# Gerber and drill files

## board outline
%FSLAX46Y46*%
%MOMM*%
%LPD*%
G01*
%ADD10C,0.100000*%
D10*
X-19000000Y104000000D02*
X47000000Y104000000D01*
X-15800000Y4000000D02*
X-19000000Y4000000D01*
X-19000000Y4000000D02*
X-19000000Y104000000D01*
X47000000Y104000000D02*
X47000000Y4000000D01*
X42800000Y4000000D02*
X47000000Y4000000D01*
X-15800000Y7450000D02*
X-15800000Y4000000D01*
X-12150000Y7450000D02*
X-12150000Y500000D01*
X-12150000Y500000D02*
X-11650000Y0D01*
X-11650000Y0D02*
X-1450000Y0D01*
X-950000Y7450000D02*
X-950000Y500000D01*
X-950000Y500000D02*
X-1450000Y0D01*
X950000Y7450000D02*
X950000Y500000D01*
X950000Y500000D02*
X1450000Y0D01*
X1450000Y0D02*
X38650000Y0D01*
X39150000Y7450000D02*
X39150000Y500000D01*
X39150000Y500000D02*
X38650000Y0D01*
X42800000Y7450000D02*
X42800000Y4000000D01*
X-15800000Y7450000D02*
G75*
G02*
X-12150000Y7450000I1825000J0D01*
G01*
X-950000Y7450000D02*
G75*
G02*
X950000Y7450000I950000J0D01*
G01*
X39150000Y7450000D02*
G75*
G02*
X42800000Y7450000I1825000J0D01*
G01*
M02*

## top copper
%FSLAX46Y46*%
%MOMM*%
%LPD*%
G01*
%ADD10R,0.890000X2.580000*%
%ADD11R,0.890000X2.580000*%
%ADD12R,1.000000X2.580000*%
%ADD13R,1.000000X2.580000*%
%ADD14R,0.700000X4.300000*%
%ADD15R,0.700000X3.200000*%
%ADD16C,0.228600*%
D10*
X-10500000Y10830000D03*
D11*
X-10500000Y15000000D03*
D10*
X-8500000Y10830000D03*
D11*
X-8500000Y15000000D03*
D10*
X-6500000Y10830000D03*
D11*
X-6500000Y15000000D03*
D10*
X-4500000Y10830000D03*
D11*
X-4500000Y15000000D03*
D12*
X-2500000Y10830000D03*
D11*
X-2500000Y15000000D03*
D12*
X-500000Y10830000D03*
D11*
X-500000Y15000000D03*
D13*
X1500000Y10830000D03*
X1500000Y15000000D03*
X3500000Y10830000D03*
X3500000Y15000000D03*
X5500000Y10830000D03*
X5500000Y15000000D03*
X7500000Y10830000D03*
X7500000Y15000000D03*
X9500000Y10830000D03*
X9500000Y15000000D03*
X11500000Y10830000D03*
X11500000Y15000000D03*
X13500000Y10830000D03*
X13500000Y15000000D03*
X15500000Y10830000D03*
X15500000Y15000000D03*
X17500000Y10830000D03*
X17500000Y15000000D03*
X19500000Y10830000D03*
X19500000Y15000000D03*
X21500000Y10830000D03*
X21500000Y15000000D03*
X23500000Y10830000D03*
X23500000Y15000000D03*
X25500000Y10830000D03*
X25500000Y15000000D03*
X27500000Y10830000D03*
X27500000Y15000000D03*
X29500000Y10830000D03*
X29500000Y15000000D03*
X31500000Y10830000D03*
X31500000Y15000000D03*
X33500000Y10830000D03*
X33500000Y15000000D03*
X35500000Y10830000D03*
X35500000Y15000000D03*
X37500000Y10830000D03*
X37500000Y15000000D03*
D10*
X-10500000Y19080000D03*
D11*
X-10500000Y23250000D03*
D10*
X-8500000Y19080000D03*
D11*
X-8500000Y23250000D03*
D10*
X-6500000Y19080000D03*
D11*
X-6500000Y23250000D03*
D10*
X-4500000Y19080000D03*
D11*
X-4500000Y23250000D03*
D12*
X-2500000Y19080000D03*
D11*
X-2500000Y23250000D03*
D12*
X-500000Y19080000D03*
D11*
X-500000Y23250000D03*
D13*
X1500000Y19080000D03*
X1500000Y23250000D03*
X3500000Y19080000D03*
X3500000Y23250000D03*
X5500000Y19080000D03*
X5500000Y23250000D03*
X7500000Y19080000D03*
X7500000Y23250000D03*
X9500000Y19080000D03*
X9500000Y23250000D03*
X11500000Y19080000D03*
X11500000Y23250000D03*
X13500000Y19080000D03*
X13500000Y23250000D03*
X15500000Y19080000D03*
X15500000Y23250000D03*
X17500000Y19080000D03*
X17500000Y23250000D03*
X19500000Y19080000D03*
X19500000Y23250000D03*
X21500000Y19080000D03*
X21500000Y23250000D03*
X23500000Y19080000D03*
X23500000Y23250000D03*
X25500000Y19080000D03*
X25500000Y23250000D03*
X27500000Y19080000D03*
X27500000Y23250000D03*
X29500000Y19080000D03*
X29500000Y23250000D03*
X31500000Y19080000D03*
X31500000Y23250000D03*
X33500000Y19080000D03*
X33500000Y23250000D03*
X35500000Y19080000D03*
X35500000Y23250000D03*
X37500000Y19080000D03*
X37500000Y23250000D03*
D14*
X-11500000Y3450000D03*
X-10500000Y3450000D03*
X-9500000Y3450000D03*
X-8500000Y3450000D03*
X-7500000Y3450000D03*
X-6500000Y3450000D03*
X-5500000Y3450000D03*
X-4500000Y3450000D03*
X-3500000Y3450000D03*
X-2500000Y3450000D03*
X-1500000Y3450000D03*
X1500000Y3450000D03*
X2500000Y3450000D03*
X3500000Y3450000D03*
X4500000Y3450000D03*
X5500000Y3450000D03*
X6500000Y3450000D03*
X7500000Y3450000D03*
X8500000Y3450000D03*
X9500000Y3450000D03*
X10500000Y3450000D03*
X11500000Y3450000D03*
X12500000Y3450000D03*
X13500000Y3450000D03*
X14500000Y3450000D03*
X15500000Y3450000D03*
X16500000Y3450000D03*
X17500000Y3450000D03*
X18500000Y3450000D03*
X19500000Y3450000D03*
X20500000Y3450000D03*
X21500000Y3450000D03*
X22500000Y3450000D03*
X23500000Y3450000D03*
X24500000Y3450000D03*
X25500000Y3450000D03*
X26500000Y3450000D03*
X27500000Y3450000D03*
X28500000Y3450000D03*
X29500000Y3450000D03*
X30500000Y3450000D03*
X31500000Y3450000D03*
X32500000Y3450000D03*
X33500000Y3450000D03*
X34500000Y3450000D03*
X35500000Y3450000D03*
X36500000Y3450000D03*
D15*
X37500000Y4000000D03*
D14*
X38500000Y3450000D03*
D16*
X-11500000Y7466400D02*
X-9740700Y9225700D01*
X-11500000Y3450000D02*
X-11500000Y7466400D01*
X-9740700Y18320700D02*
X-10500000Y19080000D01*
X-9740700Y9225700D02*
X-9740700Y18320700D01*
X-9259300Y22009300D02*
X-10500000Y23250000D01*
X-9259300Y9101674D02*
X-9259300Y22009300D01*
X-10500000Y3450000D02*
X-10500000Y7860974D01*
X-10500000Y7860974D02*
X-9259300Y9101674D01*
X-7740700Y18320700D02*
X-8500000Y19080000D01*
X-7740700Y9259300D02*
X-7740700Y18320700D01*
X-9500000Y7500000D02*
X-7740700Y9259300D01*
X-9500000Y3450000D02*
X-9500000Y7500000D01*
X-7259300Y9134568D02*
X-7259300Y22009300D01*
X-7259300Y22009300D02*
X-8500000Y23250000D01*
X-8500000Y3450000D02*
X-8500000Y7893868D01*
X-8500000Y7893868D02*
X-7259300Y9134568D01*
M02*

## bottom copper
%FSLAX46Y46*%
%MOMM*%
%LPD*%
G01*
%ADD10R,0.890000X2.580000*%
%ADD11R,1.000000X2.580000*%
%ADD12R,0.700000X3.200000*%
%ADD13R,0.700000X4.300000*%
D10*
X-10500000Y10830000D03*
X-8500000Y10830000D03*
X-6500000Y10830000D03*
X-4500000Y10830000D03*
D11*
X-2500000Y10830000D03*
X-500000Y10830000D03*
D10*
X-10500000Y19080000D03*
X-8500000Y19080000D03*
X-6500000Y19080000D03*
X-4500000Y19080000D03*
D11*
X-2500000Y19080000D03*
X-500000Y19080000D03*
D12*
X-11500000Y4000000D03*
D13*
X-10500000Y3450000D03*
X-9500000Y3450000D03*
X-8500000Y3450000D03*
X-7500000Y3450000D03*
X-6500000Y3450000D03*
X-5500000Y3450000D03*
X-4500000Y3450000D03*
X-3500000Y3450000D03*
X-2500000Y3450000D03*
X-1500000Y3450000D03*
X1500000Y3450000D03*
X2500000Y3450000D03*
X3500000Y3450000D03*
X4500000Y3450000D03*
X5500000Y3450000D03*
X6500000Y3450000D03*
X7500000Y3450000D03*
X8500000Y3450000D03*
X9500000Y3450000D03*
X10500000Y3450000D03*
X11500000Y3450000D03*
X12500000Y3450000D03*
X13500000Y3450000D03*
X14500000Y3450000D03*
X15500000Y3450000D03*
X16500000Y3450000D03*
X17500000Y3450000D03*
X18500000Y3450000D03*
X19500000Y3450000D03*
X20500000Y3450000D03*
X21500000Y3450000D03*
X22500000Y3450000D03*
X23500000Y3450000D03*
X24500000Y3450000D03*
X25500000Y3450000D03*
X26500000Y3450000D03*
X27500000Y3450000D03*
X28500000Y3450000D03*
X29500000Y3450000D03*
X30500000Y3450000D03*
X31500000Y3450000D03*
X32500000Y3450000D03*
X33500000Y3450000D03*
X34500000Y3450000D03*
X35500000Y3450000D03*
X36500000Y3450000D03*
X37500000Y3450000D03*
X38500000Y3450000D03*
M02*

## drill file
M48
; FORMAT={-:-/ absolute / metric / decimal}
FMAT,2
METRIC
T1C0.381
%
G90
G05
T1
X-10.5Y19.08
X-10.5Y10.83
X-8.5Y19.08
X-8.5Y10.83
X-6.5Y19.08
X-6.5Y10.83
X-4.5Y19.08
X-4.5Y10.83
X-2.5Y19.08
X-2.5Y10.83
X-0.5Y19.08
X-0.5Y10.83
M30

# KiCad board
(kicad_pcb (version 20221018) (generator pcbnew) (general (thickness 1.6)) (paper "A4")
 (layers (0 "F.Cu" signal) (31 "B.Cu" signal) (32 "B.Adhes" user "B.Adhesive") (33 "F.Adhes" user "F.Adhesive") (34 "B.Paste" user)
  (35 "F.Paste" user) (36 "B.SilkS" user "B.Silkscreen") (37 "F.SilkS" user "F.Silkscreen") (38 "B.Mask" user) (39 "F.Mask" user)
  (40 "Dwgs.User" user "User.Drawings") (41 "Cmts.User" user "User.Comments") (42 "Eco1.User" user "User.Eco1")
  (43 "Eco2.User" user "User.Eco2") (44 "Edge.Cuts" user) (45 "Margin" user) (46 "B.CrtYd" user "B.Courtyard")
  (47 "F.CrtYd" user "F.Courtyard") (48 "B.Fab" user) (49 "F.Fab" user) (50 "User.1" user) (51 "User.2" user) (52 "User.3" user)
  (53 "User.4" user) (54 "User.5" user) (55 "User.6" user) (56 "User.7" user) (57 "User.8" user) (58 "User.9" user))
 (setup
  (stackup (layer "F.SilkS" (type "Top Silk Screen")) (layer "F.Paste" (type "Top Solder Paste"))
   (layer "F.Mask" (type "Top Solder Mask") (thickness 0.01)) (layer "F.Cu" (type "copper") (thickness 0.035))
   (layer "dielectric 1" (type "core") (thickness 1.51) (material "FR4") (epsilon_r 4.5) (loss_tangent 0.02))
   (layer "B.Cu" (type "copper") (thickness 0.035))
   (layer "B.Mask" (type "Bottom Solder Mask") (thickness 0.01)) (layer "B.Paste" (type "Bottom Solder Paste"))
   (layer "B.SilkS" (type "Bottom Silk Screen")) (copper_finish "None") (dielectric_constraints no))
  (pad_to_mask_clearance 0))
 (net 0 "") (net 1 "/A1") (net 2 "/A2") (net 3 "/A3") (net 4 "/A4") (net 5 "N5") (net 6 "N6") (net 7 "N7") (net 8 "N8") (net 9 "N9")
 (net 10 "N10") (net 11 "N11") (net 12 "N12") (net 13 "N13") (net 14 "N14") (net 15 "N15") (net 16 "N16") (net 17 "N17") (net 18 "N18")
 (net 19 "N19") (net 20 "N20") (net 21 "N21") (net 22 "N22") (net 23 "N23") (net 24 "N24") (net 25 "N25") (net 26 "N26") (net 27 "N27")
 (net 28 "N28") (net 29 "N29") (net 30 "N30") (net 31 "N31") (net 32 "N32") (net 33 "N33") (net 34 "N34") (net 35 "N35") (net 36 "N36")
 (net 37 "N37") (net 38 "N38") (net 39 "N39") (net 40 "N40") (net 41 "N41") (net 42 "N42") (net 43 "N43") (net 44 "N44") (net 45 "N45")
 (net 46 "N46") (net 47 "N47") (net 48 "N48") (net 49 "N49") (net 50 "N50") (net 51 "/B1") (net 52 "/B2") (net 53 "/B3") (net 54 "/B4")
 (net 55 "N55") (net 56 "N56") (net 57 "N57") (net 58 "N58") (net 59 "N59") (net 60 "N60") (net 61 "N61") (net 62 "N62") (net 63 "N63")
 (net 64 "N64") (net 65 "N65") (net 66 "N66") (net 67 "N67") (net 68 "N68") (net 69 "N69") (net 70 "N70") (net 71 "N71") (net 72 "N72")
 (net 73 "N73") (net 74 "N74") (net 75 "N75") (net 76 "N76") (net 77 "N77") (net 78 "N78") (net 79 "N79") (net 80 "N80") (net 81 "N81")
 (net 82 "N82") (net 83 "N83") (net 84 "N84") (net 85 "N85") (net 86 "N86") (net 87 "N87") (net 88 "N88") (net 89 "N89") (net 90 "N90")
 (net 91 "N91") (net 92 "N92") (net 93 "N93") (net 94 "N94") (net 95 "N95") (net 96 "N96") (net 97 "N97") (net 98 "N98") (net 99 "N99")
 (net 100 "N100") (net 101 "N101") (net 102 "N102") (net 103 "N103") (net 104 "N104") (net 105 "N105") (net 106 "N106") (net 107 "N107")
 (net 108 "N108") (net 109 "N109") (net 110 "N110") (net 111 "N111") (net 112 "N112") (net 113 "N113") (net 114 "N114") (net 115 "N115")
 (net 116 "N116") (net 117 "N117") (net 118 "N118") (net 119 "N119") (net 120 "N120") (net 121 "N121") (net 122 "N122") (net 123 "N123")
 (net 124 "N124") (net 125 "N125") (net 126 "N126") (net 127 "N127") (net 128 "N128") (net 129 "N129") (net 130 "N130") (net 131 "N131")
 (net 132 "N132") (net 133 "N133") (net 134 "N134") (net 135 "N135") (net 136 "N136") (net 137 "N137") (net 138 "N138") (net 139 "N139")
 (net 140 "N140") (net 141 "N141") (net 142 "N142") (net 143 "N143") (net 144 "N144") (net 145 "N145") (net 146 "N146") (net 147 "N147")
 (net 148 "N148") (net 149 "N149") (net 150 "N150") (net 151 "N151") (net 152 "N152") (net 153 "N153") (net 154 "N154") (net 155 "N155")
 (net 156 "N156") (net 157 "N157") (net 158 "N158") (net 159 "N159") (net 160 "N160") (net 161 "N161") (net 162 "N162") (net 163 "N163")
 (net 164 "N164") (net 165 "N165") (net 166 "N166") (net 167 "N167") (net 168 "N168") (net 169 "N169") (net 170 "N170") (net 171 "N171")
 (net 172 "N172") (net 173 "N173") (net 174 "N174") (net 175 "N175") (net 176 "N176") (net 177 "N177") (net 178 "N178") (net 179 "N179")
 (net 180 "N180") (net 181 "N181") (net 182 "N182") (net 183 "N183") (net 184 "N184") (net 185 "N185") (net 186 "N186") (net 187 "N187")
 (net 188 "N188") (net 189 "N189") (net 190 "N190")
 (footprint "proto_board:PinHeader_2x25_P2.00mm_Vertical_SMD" (layer "F.Cu") (at 13.5 -12.915 90)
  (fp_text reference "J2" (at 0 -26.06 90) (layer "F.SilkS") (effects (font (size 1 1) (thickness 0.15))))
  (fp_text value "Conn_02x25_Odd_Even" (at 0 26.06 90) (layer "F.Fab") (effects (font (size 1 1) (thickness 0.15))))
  (pad "1" thru_hole rect (at -2.085 -24 90) (size 2.58 0.89) (drill 0.381) (layers "*.Cu" "*.Mask") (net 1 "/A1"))
  (pad "2" smd rect (at 2.085 -24 90) (size 2.58 0.89) (layers "F.Cu" "F.Paste" "F.Mask") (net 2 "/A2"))
  (pad "3" thru_hole rect (at -2.085 -22 90) (size 2.58 0.89) (drill 0.381) (layers "*.Cu" "*.Mask") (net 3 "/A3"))
  (pad "4" smd rect (at 2.085 -22 90) (size 2.58 0.89) (layers "F.Cu" "F.Paste" "F.Mask") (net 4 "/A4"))
  (pad "5" thru_hole rect (at -2.085 -20 90) (size 2.58 0.89) (drill 0.381) (layers "*.Cu" "*.Mask") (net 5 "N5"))
  (pad "6" smd rect (at 2.085 -20 90) (size 2.58 0.89) (layers "F.Cu" "F.Paste" "F.Mask") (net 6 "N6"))
  (pad "7" thru_hole rect (at -2.085 -18 90) (size 2.58 0.89) (drill 0.381) (layers "*.Cu" "*.Mask") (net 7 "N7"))
  (pad "8" smd rect (at 2.085 -18 90) (size 2.58 0.89) (layers "F.Cu" "F.Paste" "F.Mask") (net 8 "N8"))
  (pad "9" thru_hole rect (at -2.085 -16 90) (size 2.58 1) (drill 0.381) (layers "*.Cu" "*.Mask") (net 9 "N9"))
  (pad "10" smd rect (at 2.085 -16 90) (size 2.58 0.89) (layers "F.Cu" "F.Paste" "F.Mask") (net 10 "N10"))
  (pad "11" thru_hole rect (at -2.085 -14 90) (size 2.58 1) (drill 0.381) (layers "*.Cu" "*.Mask") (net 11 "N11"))
  (pad "12" smd rect (at 2.085 -14 90) (size 2.58 0.89) (layers "F.Cu" "F.Paste" "F.Mask") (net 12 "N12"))
  (pad "13" smd rect (at -2.085 -12 90) (size 2.58 1) (layers "F.Cu" "F.Paste" "F.Mask") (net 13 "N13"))
  (pad "14" smd rect (at 2.085 -12 90) (size 2.58 1) (layers "F.Cu" "F.Paste" "F.Mask") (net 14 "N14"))
  (pad "15" smd rect (at -2.085 -10 90) (size 2.58 1) (layers "F.Cu" "F.Paste" "F.Mask") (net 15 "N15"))
  (pad "16" smd rect (at 2.085 -10 90) (size 2.58 1) (layers "F.Cu" "F.Paste" "F.Mask") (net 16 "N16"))
  (pad "17" smd rect (at -2.085 -8 90) (size 2.58 1) (layers "F.Cu" "F.Paste" "F.Mask") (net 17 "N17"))
  (pad "18" smd rect (at 2.085 -8 90) (size 2.58 1) (layers "F.Cu" "F.Paste" "F.Mask") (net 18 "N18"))
  (pad "19" smd rect (at -2.085 -6 90) (size 2.58 1) (layers "F.Cu" "F.Paste" "F.Mask") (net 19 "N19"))
  (pad "20" smd rect (at 2.085 -6 90) (size 2.58 1) (layers "F.Cu" "F.Paste" "F.Mask") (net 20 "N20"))
  (pad "21" smd rect (at -2.085 -4 90) (size 2.58 1) (layers "F.Cu" "F.Paste" "F.Mask") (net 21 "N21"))
  (pad "22" smd rect (at 2.085 -4 90) (size 2.58 1) (layers "F.Cu" "F.Paste" "F.Mask") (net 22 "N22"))
  (pad "23" smd rect (at -2.085 -2 90) (size 2.58 1) (layers "F.Cu" "F.Paste" "F.Mask") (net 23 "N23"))
  (pad "24" smd rect (at 2.085 -2 90) (size 2.58 1) (layers "F.Cu" "F.Paste" "F.Mask") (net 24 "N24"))
  (pad "25" smd rect (at -2.085 0 90) (size 2.58 1) (layers "F.Cu" "F.Paste" "F.Mask") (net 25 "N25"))
  (pad "26" smd rect (at 2.085 0 90) (size 2.58 1) (layers "F.Cu" "F.Paste" "F.Mask") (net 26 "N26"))
  (pad "27" smd rect (at -2.085 2 90) (size 2.58 1) (layers "F.Cu" "F.Paste" "F.Mask") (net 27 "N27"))
  (pad "28" smd rect (at 2.085 2 90) (size 2.58 1) (layers "F.Cu" "F.Paste" "F.Mask") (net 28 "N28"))
  (pad "29" smd rect (at -2.085 4 90) (size 2.58 1) (layers "F.Cu" "F.Paste" "F.Mask") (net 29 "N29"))
  (pad "30" smd rect (at 2.085 4 90) (size 2.58 1) (layers "F.Cu" "F.Paste" "F.Mask") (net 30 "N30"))
  (pad "31" smd rect (at -2.085 6 90) (size 2.58 1) (layers "F.Cu" "F.Paste" "F.Mask") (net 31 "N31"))
  (pad "32" smd rect (at 2.085 6 90) (size 2.58 1) (layers "F.Cu" "F.Paste" "F.Mask") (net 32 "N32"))
  (pad "33" smd rect (at -2.085 8 90) (size 2.58 1) (layers "F.Cu" "F.Paste" "F.Mask") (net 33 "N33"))
  (pad "34" smd rect (at 2.085 8 90) (size 2.58 1) (layers "F.Cu" "F.Paste" "F.Mask") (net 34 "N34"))
  (pad "35" smd rect (at -2.085 10 90) (size 2.58 1) (layers "F.Cu" "F.Paste" "F.Mask") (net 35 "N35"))
  (pad "36" smd rect (at 2.085 10 90) (size 2.58 1) (layers "F.Cu" "F.Paste" "F.Mask") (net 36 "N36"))
  (pad "37" smd rect (at -2.085 12 90) (size 2.58 1) (layers "F.Cu" "F.Paste" "F.Mask") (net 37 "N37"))
  (pad "38" smd rect (at 2.085 12 90) (size 2.58 1) (layers "F.Cu" "F.Paste" "F.Mask") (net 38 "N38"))
  (pad "39" smd rect (at -2.085 14 90) (size 2.58 1) (layers "F.Cu" "F.Paste" "F.Mask") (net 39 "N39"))
  (pad "40" smd rect (at 2.085 14 90) (size 2.58 1) (layers "F.Cu" "F.Paste" "F.Mask") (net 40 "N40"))
  (pad "41" smd rect (at -2.085 16 90) (size 2.58 1) (layers "F.Cu" "F.Paste" "F.Mask") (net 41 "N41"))
  (pad "42" smd rect (at 2.085 16 90) (size 2.58 1) (layers "F.Cu" "F.Paste" "F.Mask") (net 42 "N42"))
  (pad "43" smd rect (at -2.085 18 90) (size 2.58 1) (layers "F.Cu" "F.Paste" "F.Mask") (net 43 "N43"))
  (pad "44" smd rect (at 2.085 18 90) (size 2.58 1) (layers "F.Cu" "F.Paste" "F.Mask") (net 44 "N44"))
  (pad "45" smd rect (at -2.085 20 90) (size 2.58 1) (layers "F.Cu" "F.Paste" "F.Mask") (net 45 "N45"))
  (pad "46" smd rect (at 2.085 20 90) (size 2.58 1) (layers "F.Cu" "F.Paste" "F.Mask") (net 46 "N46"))
  (pad "47" smd rect (at -2.085 22 90) (size 2.58 1) (layers "F.Cu" "F.Paste" "F.Mask") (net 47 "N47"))
  (pad "48" smd rect (at 2.085 22 90) (size 2.58 1) (layers "F.Cu" "F.Paste" "F.Mask") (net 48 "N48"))
  (pad "49" smd rect (at -2.085 24 90) (size 2.58 1) (layers "F.Cu" "F.Paste" "F.Mask") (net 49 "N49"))
  (pad "50" smd rect (at 2.085 24 90) (size 2.58 1) (layers "F.Cu" "F.Paste" "F.Mask") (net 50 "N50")))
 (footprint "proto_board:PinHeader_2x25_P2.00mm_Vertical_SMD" (layer "F.Cu") (at 13.5 -21.165 90)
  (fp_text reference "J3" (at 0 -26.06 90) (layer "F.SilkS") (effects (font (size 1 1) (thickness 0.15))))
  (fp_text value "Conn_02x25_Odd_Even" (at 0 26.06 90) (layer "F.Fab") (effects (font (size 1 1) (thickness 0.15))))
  (pad "1" thru_hole rect (at -2.085 -24 90) (size 2.58 0.89) (drill 0.381) (layers "*.Cu" "*.Mask") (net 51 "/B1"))
  (pad "2" smd rect (at 2.085 -24 90) (size 2.58 0.89) (layers "F.Cu" "F.Paste" "F.Mask") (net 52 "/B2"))
  (pad "3" thru_hole rect (at -2.085 -22 90) (size 2.58 0.89) (drill 0.381) (layers "*.Cu" "*.Mask") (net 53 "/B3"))
  (pad "4" smd rect (at 2.085 -22 90) (size 2.58 0.89) (layers "F.Cu" "F.Paste" "F.Mask") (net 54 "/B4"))
  (pad "5" thru_hole rect (at -2.085 -20 90) (size 2.58 0.89) (drill 0.381) (layers "*.Cu" "*.Mask") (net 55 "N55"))
  (pad "6" smd rect (at 2.085 -20 90) (size 2.58 0.89) (layers "F.Cu" "F.Paste" "F.Mask") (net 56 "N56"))
  (pad "7" thru_hole rect (at -2.085 -18 90) (size 2.58 0.89) (drill 0.381) (layers "*.Cu" "*.Mask") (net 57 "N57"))
  (pad "8" smd rect (at 2.085 -18 90) (size 2.58 0.89) (layers "F.Cu" "F.Paste" "F.Mask") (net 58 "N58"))
  (pad "9" thru_hole rect (at -2.085 -16 90) (size 2.58 1) (drill 0.381) (layers "*.Cu" "*.Mask") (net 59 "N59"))
  (pad "10" smd rect (at 2.085 -16 90) (size 2.58 0.89) (layers "F.Cu" "F.Paste" "F.Mask") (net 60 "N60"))
  (pad "11" thru_hole rect (at -2.085 -14 90) (size 2.58 1) (drill 0.381) (layers "*.Cu" "*.Mask") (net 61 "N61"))
  (pad "12" smd rect (at 2.085 -14 90) (size 2.58 0.89) (layers "F.Cu" "F.Paste" "F.Mask") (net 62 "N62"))
  (pad "13" smd rect (at -2.085 -12 90) (size 2.58 1) (layers "F.Cu" "F.Paste" "F.Mask") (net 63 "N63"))
  (pad "14" smd rect (at 2.085 -12 90) (size 2.58 1) (layers "F.Cu" "F.Paste" "F.Mask") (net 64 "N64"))
  (pad "15" smd rect (at -2.085 -10 90) (size 2.58 1) (layers "F.Cu" "F.Paste" "F.Mask") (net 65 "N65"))
  (pad "16" smd rect (at 2.085 -10 90) (size 2.58 1) (layers "F.Cu" "F.Paste" "F.Mask") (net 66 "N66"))
  (pad "17" smd rect (at -2.085 -8 90) (size 2.58 1) (layers "F.Cu" "F.Paste" "F.Mask") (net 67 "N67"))
  (pad "18" smd rect (at 2.085 -8 90) (size 2.58 1) (layers "F.Cu" "F.Paste" "F.Mask") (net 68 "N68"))
  (pad "19" smd rect (at -2.085 -6 90) (size 2.58 1) (layers "F.Cu" "F.Paste" "F.Mask") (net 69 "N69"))
  (pad "20" smd rect (at 2.085 -6 90) (size 2.58 1) (layers "F.Cu" "F.Paste" "F.Mask") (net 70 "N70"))
  (pad "21" smd rect (at -2.085 -4 90) (size 2.58 1) (layers "F.Cu" "F.Paste" "F.Mask") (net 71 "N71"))
  (pad "22" smd rect (at 2.085 -4 90) (size 2.58 1) (layers "F.Cu" "F.Paste" "F.Mask") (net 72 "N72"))
  (pad "23" smd rect (at -2.085 -2 90) (size 2.58 1) (layers "F.Cu" "F.Paste" "F.Mask") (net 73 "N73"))
  (pad "24" smd rect (at 2.085 -2 90) (size 2.58 1) (layers "F.Cu" "F.Paste" "F.Mask") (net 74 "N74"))
  (pad "25" smd rect (at -2.085 0 90) (size 2.58 1) (layers "F.Cu" "F.Paste" "F.Mask") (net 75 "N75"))
  (pad "26" smd rect (at 2.085 0 90) (size 2.58 1) (layers "F.Cu" "F.Paste" "F.Mask") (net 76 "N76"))
  (pad "27" smd rect (at -2.085 2 90) (size 2.58 1) (layers "F.Cu" "F.Paste" "F.Mask") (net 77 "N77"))
  (pad "28" smd rect (at 2.085 2 90) (size 2.58 1) (layers "F.Cu" "F.Paste" "F.Mask") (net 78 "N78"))
  (pad "29" smd rect (at -2.085 4 90) (size 2.58 1) (layers "F.Cu" "F.Paste" "F.Mask") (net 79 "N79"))
  (pad "30" smd rect (at 2.085 4 90) (size 2.58 1) (layers "F.Cu" "F.Paste" "F.Mask") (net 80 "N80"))
  (pad "31" smd rect (at -2.085 6 90) (size 2.58 1) (layers "F.Cu" "F.Paste" "F.Mask") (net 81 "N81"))
  (pad "32" smd rect (at 2.085 6 90) (size 2.58 1) (layers "F.Cu" "F.Paste" "F.Mask") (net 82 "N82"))
  (pad "33" smd rect (at -2.085 8 90) (size 2.58 1) (layers "F.Cu" "F.Paste" "F.Mask") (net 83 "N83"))
  (pad "34" smd rect (at 2.085 8 90) (size 2.58 1) (layers "F.Cu" "F.Paste" "F.Mask") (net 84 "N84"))
  (pad "35" smd rect (at -2.085 10 90) (size 2.58 1) (layers "F.Cu" "F.Paste" "F.Mask") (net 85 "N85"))
  (pad "36" smd rect (at 2.085 10 90) (size 2.58 1) (layers "F.Cu" "F.Paste" "F.Mask") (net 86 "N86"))
  (pad "37" smd rect (at -2.085 12 90) (size 2.58 1) (layers "F.Cu" "F.Paste" "F.Mask") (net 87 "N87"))
  (pad "38" smd rect (at 2.085 12 90) (size 2.58 1) (layers "F.Cu" "F.Paste" "F.Mask") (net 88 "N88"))
  (pad "39" smd rect (at -2.085 14 90) (size 2.58 1) (layers "F.Cu" "F.Paste" "F.Mask") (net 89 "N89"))
  (pad "40" smd rect (at 2.085 14 90) (size 2.58 1) (layers "F.Cu" "F.Paste" "F.Mask") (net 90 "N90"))
  (pad "41" smd rect (at -2.085 16 90) (size 2.58 1) (layers "F.Cu" "F.Paste" "F.Mask") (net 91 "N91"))
  (pad "42" smd rect (at 2.085 16 90) (size 2.58 1) (layers "F.Cu" "F.Paste" "F.Mask") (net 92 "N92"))
  (pad "43" smd rect (at -2.085 18 90) (size 2.58 1) (layers "F.Cu" "F.Paste" "F.Mask") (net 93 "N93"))
  (pad "44" smd rect (at 2.085 18 90) (size 2.58 1) (layers "F.Cu" "F.Paste" "F.Mask") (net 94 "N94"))
  (pad "45" smd rect (at -2.085 20 90) (size 2.58 1) (layers "F.Cu" "F.Paste" "F.Mask") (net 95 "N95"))
  (pad "46" smd rect (at 2.085 20 90) (size 2.58 1) (layers "F.Cu" "F.Paste" "F.Mask") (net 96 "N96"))
  (pad "47" smd rect (at -2.085 22 90) (size 2.58 1) (layers "F.Cu" "F.Paste" "F.Mask") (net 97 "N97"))
  (pad "48" smd rect (at 2.085 22 90) (size 2.58 1) (layers "F.Cu" "F.Paste" "F.Mask") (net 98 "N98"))
  (pad "49" smd rect (at -2.085 24 90) (size 2.58 1) (layers "F.Cu" "F.Paste" "F.Mask") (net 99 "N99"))
  (pad "50" smd rect (at 2.085 24 90) (size 2.58 1) (layers "F.Cu" "F.Paste" "F.Mask") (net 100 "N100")))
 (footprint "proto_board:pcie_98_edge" (layer "F.Cu") (at 0 0)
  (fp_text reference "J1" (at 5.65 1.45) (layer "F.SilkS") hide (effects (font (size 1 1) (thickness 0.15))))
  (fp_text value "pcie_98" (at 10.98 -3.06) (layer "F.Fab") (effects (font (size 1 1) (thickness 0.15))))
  (fp_line (start -15.8 -7.45) (end -15.8 -4) (stroke (width 0.1) (type solid)) (layer "Edge.Cuts"))
  (fp_line (start -12.15 -7.45) (end -12.15 -0.5) (stroke (width 0.1) (type solid)) (layer "Edge.Cuts"))
  (fp_line (start -12.15 -0.5) (end -11.65 0) (stroke (width 0.1) (type solid)) (layer "Edge.Cuts"))
  (fp_line (start -11.65 0) (end -1.45 0) (stroke (width 0.1) (type solid)) (layer "Edge.Cuts"))
  (fp_line (start -0.95 -7.45) (end -0.95 -0.5) (stroke (width 0.1) (type solid)) (layer "Edge.Cuts"))
  (fp_line (start -0.95 -0.5) (end -1.45 0) (stroke (width 0.1) (type solid)) (layer "Edge.Cuts"))
  (fp_line (start 0.95 -7.45) (end 0.95 -0.5) (stroke (width 0.1) (type solid)) (layer "Edge.Cuts"))
  (fp_line (start 0.95 -0.5) (end 1.45 0) (stroke (width 0.1) (type solid)) (layer "Edge.Cuts"))
  (fp_line (start 1.45 0) (end 38.65 0) (stroke (width 0.1) (type solid)) (layer "Edge.Cuts"))
  (fp_line (start 39.15 -7.45) (end 39.15 -0.5) (stroke (width 0.1) (type solid)) (layer "Edge.Cuts"))
  (fp_line (start 39.15 -0.5) (end 38.65 0) (stroke (width 0.1) (type solid)) (layer "Edge.Cuts"))
  (fp_line (start 42.8 -7.45) (end 42.8 -4) (stroke (width 0.1) (type solid)) (layer "Edge.Cuts"))
  (fp_arc (start -15.8 -7.45) (mid -13.975 -9.275) (end -12.15 -7.45) (stroke (width 0.1) (type default)) (layer "Edge.Cuts"))
  (fp_arc (start -0.95 -7.45) (mid 0 -8.4) (end 0.95 -7.45) (stroke (width 0.1) (type solid)) (layer "Edge.Cuts"))
  (fp_arc (start 39.15 -7.45) (mid 40.975 -9.275) (end 42.8 -7.45) (stroke (width 0.1) (type default)) (layer "Edge.Cuts"))
  (pad "A1" connect rect (at -11.5 -4) (size 0.7 3.2) (layers "B.Cu" "B.Mask") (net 1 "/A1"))
  (pad "A2" connect rect (at -10.5 -3.45) (size 0.7 4.3) (layers "B.Cu" "B.Mask") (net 2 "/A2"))
  (pad "A3" connect rect (at -9.5 -3.45) (size 0.7 4.3) (layers "B.Cu" "B.Mask") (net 3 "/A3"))
  (pad "A4" connect rect (at -8.5 -3.45) (size 0.7 4.3) (layers "B.Cu" "B.Mask") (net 4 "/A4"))
  (pad "A5" connect rect (at -7.5 -3.45) (size 0.7 4.3) (layers "B.Cu" "B.Mask") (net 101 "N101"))
  (pad "A6" connect rect (at -6.5 -3.45) (size 0.7 4.3) (layers "B.Cu" "B.Mask") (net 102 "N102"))
  (pad "A7" connect rect (at -5.5 -3.45) (size 0.7 4.3) (layers "B.Cu" "B.Mask") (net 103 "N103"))
  (pad "A8" connect rect (at -4.5 -3.45) (size 0.7 4.3) (layers "B.Cu" "B.Mask") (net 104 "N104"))
  (pad "A9" connect rect (at -3.5 -3.45) (size 0.7 4.3) (layers "B.Cu" "B.Mask") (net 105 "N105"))
  (pad "A10" connect rect (at -2.5 -3.45) (size 0.7 4.3) (layers "B.Cu" "B.Mask") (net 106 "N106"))
  (pad "A11" connect rect (at -1.5 -3.45) (size 0.7 4.3) (layers "B.Cu" "B.Mask") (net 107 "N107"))
  (pad "A12" connect rect (at 1.5 -3.45) (size 0.7 4.3) (layers "B.Cu" "B.Mask") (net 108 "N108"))
  (pad "A13" connect rect (at 2.5 -3.45) (size 0.7 4.3) (layers "B.Cu" "B.Mask") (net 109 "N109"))
  (pad "A14" connect rect (at 3.5 -3.45) (size 0.7 4.3) (layers "B.Cu" "B.Mask") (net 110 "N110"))
  (pad "A15" connect rect (at 4.5 -3.45) (size 0.7 4.3) (layers "B.Cu" "B.Mask") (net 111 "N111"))
  (pad "A16" connect rect (at 5.5 -3.45) (size 0.7 4.3) (layers "B.Cu" "B.Mask") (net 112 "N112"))
  (pad "A17" connect rect (at 6.5 -3.45) (size 0.7 4.3) (layers "B.Cu" "B.Mask") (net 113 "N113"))
  (pad "A18" connect rect (at 7.5 -3.45) (size 0.7 4.3) (layers "B.Cu" "B.Mask") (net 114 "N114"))
  (pad "A19" connect rect (at 8.5 -3.45) (size 0.7 4.3) (layers "B.Cu" "B.Mask") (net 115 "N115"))
  (pad "A20" connect rect (at 9.5 -3.45) (size 0.7 4.3) (layers "B.Cu" "B.Mask") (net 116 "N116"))
  (pad "A21" connect rect (at 10.5 -3.45) (size 0.7 4.3) (layers "B.Cu" "B.Mask") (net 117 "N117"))
  (pad "A22" connect rect (at 11.5 -3.45) (size 0.7 4.3) (layers "B.Cu" "B.Mask") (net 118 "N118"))
  (pad "A23" connect rect (at 12.5 -3.45) (size 0.7 4.3) (layers "B.Cu" "B.Mask") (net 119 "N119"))
  (pad "A24" connect rect (at 13.5 -3.45) (size 0.7 4.3) (layers "B.Cu" "B.Mask") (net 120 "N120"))
  (pad "A25" connect rect (at 14.5 -3.45) (size 0.7 4.3) (layers "B.Cu" "B.Mask") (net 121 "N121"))
  (pad "A26" connect rect (at 15.5 -3.45) (size 0.7 4.3) (layers "B.Cu" "B.Mask") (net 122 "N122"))
  (pad "A27" connect rect (at 16.5 -3.45) (size 0.7 4.3) (layers "B.Cu" "B.Mask") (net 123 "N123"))
  (pad "A28" connect rect (at 17.5 -3.45) (size 0.7 4.3) (layers "B.Cu" "B.Mask") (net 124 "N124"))
  (pad "A29" connect rect (at 18.5 -3.45) (size 0.7 4.3) (layers "B.Cu" "B.Mask") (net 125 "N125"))
  (pad "A30" connect rect (at 19.5 -3.45) (size 0.7 4.3) (layers "B.Cu" "B.Mask") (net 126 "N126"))
  (pad "A31" connect rect (at 20.5 -3.45) (size 0.7 4.3) (layers "B.Cu" "B.Mask") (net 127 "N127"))
  (pad "A32" connect rect (at 21.5 -3.45) (size 0.7 4.3) (layers "B.Cu" "B.Mask") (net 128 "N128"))
  (pad "A33" connect rect (at 22.5 -3.45) (size 0.7 4.3) (layers "B.Cu" "B.Mask") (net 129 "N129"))
  (pad "A34" connect rect (at 23.5 -3.45) (size 0.7 4.3) (layers "B.Cu" "B.Mask") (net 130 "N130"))
  (pad "A35" connect rect (at 24.5 -3.45) (size 0.7 4.3) (layers "B.Cu" "B.Mask") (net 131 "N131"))
  (pad "A36" connect rect (at 25.5 -3.45) (size 0.7 4.3) (layers "B.Cu" "B.Mask") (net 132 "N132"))
  (pad "A37" connect rect (at 26.5 -3.45) (size 0.7 4.3) (layers "B.Cu" "B.Mask") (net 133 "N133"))
  (pad "A38" connect rect (at 27.5 -3.45) (size 0.7 4.3) (layers "B.Cu" "B.Mask") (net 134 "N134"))
  (pad "A39" connect rect (at 28.5 -3.45) (size 0.7 4.3) (layers "B.Cu" "B.Mask") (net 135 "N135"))
  (pad "A40" connect rect (at 29.5 -3.45) (size 0.7 4.3) (layers "B.Cu" "B.Mask") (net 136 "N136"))
  (pad "A41" connect rect (at 30.5 -3.45) (size 0.7 4.3) (layers "B.Cu" "B.Mask") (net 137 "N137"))
  (pad "A42" connect rect (at 31.5 -3.45) (size 0.7 4.3) (layers "B.Cu" "B.Mask") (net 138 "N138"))
  (pad "A43" connect rect (at 32.5 -3.45) (size 0.7 4.3) (layers "B.Cu" "B.Mask") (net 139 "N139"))
  (pad "A44" connect rect (at 33.5 -3.45) (size 0.7 4.3) (layers "B.Cu" "B.Mask") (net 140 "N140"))
  (pad "A45" connect rect (at 34.5 -3.45) (size 0.7 4.3) (layers "B.Cu" "B.Mask") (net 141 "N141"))
  (pad "A46" connect rect (at 35.5 -3.45) (size 0.7 4.3) (layers "B.Cu" "B.Mask") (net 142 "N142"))
  (pad "A47" connect rect (at 36.5 -3.45) (size 0.7 4.3) (layers "B.Cu" "B.Mask") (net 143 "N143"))
  (pad "A48" connect rect (at 37.5 -3.45) (size 0.7 4.3) (layers "B.Cu" "B.Mask") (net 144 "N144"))
  (pad "A49" connect rect (at 38.5 -3.45) (size 0.7 4.3) (layers "B.Cu" "B.Mask") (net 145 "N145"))
  (pad "B1" connect rect (at -11.5 -3.45) (size 0.7 4.3) (layers "F.Cu" "F.Mask") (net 51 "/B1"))
  (pad "B2" connect rect (at -10.5 -3.45) (size 0.7 4.3) (layers "F.Cu" "F.Mask") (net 52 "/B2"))
  (pad "B3" connect rect (at -9.5 -3.45) (size 0.7 4.3) (layers "F.Cu" "F.Mask") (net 53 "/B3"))
  (pad "B4" connect rect (at -8.5 -3.45) (size 0.7 4.3) (layers "F.Cu" "F.Mask") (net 54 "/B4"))
  (pad "B5" connect rect (at -7.5 -3.45) (size 0.7 4.3) (layers "F.Cu" "F.Mask") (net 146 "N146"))
  (pad "B6" connect rect (at -6.5 -3.45) (size 0.7 4.3) (layers "F.Cu" "F.Mask") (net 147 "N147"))
  (pad "B7" connect rect (at -5.5 -3.45) (size 0.7 4.3) (layers "F.Cu" "F.Mask") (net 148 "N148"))
  (pad "B8" connect rect (at -4.5 -3.45) (size 0.7 4.3) (layers "F.Cu" "F.Mask") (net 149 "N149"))
  (pad "B9" connect rect (at -3.5 -3.45) (size 0.7 4.3) (layers "F.Cu" "F.Mask") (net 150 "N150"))
  (pad "B10" connect rect (at -2.5 -3.45) (size 0.7 4.3) (layers "F.Cu" "F.Mask") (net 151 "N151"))
  (pad "B11" connect rect (at -1.5 -3.45) (size 0.7 4.3) (layers "F.Cu" "F.Mask") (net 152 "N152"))
  (pad "B12" connect rect (at 1.5 -3.45) (size 0.7 4.3) (layers "F.Cu" "F.Mask") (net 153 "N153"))
  (pad "B13" connect rect (at 2.5 -3.45) (size 0.7 4.3) (layers "F.Cu" "F.Mask") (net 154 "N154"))
  (pad "B14" connect rect (at 3.5 -3.45) (size 0.7 4.3) (layers "F.Cu" "F.Mask") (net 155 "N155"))
  (pad "B15" connect rect (at 4.5 -3.45) (size 0.7 4.3) (layers "F.Cu" "F.Mask") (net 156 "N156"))
  (pad "B16" connect rect (at 5.5 -3.45) (size 0.7 4.3) (layers "F.Cu" "F.Mask") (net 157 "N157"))
  (pad "B17" connect rect (at 6.5 -3.45) (size 0.7 4.3) (layers "F.Cu" "F.Mask") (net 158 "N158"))
  (pad "B18" connect rect (at 7.5 -3.45) (size 0.7 4.3) (layers "F.Cu" "F.Mask") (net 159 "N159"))
  (pad "B19" connect rect (at 8.5 -3.45) (size 0.7 4.3) (layers "F.Cu" "F.Mask") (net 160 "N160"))
  (pad "B20" connect rect (at 9.5 -3.45) (size 0.7 4.3) (layers "F.Cu" "F.Mask") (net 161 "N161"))
  (pad "B21" connect rect (at 10.5 -3.45) (size 0.7 4.3) (layers "F.Cu" "F.Mask") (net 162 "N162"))
  (pad "B22" connect rect (at 11.5 -3.45) (size 0.7 4.3) (layers "F.Cu" "F.Mask") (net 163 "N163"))
  (pad "B23" connect rect (at 12.5 -3.45) (size 0.7 4.3) (layers "F.Cu" "F.Mask") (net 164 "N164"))
  (pad "B24" connect rect (at 13.5 -3.45) (size 0.7 4.3) (layers "F.Cu" "F.Mask") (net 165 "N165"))
  (pad "B25" connect rect (at 14.5 -3.45) (size 0.7 4.3) (layers "F.Cu" "F.Mask") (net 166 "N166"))
  (pad "B26" connect rect (at 15.5 -3.45) (size 0.7 4.3) (layers "F.Cu" "F.Mask") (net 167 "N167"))
  (pad "B27" connect rect (at 16.5 -3.45) (size 0.7 4.3) (layers "F.Cu" "F.Mask") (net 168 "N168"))
  (pad "B28" connect rect (at 17.5 -3.45) (size 0.7 4.3) (layers "F.Cu" "F.Mask") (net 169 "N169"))
  (pad "B29" connect rect (at 18.5 -3.45) (size 0.7 4.3) (layers "F.Cu" "F.Mask") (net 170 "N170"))
  (pad "B30" connect rect (at 19.5 -3.45) (size 0.7 4.3) (layers "F.Cu" "F.Mask") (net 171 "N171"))
  (pad "B31" connect rect (at 20.5 -3.45) (size 0.7 4.3) (layers "F.Cu" "F.Mask") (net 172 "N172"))
  (pad "B32" connect rect (at 21.5 -3.45) (size 0.7 4.3) (layers "F.Cu" "F.Mask") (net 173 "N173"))
  (pad "B33" connect rect (at 22.5 -3.45) (size 0.7 4.3) (layers "F.Cu" "F.Mask") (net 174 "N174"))
  (pad "B34" connect rect (at 23.5 -3.45) (size 0.7 4.3) (layers "F.Cu" "F.Mask") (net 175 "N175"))
  (pad "B35" connect rect (at 24.5 -3.45) (size 0.7 4.3) (layers "F.Cu" "F.Mask") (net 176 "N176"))
  (pad "B36" connect rect (at 25.5 -3.45) (size 0.7 4.3) (layers "F.Cu" "F.Mask") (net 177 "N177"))
  (pad "B37" connect rect (at 26.5 -3.45) (size 0.7 4.3) (layers "F.Cu" "F.Mask") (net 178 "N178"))
  (pad "B38" connect rect (at 27.5 -3.45) (size 0.7 4.3) (layers "F.Cu" "F.Mask") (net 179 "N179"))
  (pad "B39" connect rect (at 28.5 -3.45) (size 0.7 4.3) (layers "F.Cu" "F.Mask") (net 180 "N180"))
  (pad "B40" connect rect (at 29.5 -3.45) (size 0.7 4.3) (layers "F.Cu" "F.Mask") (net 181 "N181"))
  (pad "B41" connect rect (at 30.5 -3.45) (size 0.7 4.3) (layers "F.Cu" "F.Mask") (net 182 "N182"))
  (pad "B42" connect rect (at 31.5 -3.45) (size 0.7 4.3) (layers "F.Cu" "F.Mask") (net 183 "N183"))
  (pad "B43" connect rect (at 32.5 -3.45) (size 0.7 4.3) (layers "F.Cu" "F.Mask") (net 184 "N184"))
  (pad "B44" connect rect (at 33.5 -3.45) (size 0.7 4.3) (layers "F.Cu" "F.Mask") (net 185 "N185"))
  (pad "B45" connect rect (at 34.5 -3.45) (size 0.7 4.3) (layers "F.Cu" "F.Mask") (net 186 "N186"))
  (pad "B46" connect rect (at 35.5 -3.45) (size 0.7 4.3) (layers "F.Cu" "F.Mask") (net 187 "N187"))
  (pad "B47" connect rect (at 36.5 -3.45) (size 0.7 4.3) (layers "F.Cu" "F.Mask") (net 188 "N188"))
  (pad "B48" connect rect (at 37.5 -4) (size 0.7 3.2) (layers "F.Cu" "F.Mask") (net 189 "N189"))
  (pad "B49" connect rect (at 38.5 -3.45) (size 0.7 4.3) (layers "F.Cu" "F.Mask") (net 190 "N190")))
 (gr_line (start -19 -104) (end 47 -104) (stroke (width 0.1) (type default)) (layer "Edge.Cuts"))
 (gr_line (start -15.8 -4) (end -19 -4) (stroke (width 0.1) (type default)) (layer "Edge.Cuts"))
 (gr_line (start -19 -4) (end -19 -104) (stroke (width 0.1) (type default)) (layer "Edge.Cuts"))
 (gr_line (start 47 -104) (end 47 -4) (stroke (width 0.1) (type default)) (layer "Edge.Cuts"))
 (gr_line (start 42.8 -4) (end 47 -4) (stroke (width 0.1) (type default)) (layer "Edge.Cuts"))
 (segment (start -11.5 -7.4664) (end -9.7407 -9.2257) (width 0.2286) (layer "F.Cu") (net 51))
 (segment (start -11.5 -3.45) (end -11.5 -7.4664) (width 0.2286) (layer "F.Cu") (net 51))
 (segment (start -9.7407 -18.3207) (end -10.5 -19.08) (width 0.2286) (layer "F.Cu") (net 51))
 (segment (start -9.7407 -9.2257) (end -9.7407 -18.3207) (width 0.2286) (layer "F.Cu") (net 51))
 (segment (start -9.2593 -22.0093) (end -10.5 -23.25) (width 0.2286) (layer "F.Cu") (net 52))
 (segment (start -9.2593 -9.101674) (end -9.2593 -22.0093) (width 0.2286) (layer "F.Cu") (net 52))
 (segment (start -10.5 -3.45) (end -10.5 -7.860974) (width 0.2286) (layer "F.Cu") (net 52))
 (segment (start -10.5 -7.860974) (end -9.2593 -9.101674) (width 0.2286) (layer "F.Cu") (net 52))
 (segment (start -7.7407 -18.3207) (end -8.5 -19.08) (width 0.2286) (layer "F.Cu") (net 53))
 (segment (start -7.7407 -9.2593) (end -7.7407 -18.3207) (width 0.2286) (layer "F.Cu") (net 53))
 (segment (start -9.5 -7.5) (end -7.7407 -9.2593) (width 0.2286) (layer "F.Cu") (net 53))
 (segment (start -9.5 -3.45) (end -9.5 -7.5) (width 0.2286) (layer "F.Cu") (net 53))
 (segment (start -7.2593 -9.134568) (end -7.2593 -22.0093) (width 0.2286) (layer "F.Cu") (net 54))
 (segment (start -7.2593 -22.0093) (end -8.5 -23.25) (width 0.2286) (layer "F.Cu") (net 54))
 (segment (start -8.5 -3.45) (end -8.5 -7.893868) (width 0.2286) (layer "F.Cu") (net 54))
 (segment (start -8.5 -7.893868) (end -7.2593 -9.134568) (width 0.2286) (layer "F.Cu") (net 54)))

